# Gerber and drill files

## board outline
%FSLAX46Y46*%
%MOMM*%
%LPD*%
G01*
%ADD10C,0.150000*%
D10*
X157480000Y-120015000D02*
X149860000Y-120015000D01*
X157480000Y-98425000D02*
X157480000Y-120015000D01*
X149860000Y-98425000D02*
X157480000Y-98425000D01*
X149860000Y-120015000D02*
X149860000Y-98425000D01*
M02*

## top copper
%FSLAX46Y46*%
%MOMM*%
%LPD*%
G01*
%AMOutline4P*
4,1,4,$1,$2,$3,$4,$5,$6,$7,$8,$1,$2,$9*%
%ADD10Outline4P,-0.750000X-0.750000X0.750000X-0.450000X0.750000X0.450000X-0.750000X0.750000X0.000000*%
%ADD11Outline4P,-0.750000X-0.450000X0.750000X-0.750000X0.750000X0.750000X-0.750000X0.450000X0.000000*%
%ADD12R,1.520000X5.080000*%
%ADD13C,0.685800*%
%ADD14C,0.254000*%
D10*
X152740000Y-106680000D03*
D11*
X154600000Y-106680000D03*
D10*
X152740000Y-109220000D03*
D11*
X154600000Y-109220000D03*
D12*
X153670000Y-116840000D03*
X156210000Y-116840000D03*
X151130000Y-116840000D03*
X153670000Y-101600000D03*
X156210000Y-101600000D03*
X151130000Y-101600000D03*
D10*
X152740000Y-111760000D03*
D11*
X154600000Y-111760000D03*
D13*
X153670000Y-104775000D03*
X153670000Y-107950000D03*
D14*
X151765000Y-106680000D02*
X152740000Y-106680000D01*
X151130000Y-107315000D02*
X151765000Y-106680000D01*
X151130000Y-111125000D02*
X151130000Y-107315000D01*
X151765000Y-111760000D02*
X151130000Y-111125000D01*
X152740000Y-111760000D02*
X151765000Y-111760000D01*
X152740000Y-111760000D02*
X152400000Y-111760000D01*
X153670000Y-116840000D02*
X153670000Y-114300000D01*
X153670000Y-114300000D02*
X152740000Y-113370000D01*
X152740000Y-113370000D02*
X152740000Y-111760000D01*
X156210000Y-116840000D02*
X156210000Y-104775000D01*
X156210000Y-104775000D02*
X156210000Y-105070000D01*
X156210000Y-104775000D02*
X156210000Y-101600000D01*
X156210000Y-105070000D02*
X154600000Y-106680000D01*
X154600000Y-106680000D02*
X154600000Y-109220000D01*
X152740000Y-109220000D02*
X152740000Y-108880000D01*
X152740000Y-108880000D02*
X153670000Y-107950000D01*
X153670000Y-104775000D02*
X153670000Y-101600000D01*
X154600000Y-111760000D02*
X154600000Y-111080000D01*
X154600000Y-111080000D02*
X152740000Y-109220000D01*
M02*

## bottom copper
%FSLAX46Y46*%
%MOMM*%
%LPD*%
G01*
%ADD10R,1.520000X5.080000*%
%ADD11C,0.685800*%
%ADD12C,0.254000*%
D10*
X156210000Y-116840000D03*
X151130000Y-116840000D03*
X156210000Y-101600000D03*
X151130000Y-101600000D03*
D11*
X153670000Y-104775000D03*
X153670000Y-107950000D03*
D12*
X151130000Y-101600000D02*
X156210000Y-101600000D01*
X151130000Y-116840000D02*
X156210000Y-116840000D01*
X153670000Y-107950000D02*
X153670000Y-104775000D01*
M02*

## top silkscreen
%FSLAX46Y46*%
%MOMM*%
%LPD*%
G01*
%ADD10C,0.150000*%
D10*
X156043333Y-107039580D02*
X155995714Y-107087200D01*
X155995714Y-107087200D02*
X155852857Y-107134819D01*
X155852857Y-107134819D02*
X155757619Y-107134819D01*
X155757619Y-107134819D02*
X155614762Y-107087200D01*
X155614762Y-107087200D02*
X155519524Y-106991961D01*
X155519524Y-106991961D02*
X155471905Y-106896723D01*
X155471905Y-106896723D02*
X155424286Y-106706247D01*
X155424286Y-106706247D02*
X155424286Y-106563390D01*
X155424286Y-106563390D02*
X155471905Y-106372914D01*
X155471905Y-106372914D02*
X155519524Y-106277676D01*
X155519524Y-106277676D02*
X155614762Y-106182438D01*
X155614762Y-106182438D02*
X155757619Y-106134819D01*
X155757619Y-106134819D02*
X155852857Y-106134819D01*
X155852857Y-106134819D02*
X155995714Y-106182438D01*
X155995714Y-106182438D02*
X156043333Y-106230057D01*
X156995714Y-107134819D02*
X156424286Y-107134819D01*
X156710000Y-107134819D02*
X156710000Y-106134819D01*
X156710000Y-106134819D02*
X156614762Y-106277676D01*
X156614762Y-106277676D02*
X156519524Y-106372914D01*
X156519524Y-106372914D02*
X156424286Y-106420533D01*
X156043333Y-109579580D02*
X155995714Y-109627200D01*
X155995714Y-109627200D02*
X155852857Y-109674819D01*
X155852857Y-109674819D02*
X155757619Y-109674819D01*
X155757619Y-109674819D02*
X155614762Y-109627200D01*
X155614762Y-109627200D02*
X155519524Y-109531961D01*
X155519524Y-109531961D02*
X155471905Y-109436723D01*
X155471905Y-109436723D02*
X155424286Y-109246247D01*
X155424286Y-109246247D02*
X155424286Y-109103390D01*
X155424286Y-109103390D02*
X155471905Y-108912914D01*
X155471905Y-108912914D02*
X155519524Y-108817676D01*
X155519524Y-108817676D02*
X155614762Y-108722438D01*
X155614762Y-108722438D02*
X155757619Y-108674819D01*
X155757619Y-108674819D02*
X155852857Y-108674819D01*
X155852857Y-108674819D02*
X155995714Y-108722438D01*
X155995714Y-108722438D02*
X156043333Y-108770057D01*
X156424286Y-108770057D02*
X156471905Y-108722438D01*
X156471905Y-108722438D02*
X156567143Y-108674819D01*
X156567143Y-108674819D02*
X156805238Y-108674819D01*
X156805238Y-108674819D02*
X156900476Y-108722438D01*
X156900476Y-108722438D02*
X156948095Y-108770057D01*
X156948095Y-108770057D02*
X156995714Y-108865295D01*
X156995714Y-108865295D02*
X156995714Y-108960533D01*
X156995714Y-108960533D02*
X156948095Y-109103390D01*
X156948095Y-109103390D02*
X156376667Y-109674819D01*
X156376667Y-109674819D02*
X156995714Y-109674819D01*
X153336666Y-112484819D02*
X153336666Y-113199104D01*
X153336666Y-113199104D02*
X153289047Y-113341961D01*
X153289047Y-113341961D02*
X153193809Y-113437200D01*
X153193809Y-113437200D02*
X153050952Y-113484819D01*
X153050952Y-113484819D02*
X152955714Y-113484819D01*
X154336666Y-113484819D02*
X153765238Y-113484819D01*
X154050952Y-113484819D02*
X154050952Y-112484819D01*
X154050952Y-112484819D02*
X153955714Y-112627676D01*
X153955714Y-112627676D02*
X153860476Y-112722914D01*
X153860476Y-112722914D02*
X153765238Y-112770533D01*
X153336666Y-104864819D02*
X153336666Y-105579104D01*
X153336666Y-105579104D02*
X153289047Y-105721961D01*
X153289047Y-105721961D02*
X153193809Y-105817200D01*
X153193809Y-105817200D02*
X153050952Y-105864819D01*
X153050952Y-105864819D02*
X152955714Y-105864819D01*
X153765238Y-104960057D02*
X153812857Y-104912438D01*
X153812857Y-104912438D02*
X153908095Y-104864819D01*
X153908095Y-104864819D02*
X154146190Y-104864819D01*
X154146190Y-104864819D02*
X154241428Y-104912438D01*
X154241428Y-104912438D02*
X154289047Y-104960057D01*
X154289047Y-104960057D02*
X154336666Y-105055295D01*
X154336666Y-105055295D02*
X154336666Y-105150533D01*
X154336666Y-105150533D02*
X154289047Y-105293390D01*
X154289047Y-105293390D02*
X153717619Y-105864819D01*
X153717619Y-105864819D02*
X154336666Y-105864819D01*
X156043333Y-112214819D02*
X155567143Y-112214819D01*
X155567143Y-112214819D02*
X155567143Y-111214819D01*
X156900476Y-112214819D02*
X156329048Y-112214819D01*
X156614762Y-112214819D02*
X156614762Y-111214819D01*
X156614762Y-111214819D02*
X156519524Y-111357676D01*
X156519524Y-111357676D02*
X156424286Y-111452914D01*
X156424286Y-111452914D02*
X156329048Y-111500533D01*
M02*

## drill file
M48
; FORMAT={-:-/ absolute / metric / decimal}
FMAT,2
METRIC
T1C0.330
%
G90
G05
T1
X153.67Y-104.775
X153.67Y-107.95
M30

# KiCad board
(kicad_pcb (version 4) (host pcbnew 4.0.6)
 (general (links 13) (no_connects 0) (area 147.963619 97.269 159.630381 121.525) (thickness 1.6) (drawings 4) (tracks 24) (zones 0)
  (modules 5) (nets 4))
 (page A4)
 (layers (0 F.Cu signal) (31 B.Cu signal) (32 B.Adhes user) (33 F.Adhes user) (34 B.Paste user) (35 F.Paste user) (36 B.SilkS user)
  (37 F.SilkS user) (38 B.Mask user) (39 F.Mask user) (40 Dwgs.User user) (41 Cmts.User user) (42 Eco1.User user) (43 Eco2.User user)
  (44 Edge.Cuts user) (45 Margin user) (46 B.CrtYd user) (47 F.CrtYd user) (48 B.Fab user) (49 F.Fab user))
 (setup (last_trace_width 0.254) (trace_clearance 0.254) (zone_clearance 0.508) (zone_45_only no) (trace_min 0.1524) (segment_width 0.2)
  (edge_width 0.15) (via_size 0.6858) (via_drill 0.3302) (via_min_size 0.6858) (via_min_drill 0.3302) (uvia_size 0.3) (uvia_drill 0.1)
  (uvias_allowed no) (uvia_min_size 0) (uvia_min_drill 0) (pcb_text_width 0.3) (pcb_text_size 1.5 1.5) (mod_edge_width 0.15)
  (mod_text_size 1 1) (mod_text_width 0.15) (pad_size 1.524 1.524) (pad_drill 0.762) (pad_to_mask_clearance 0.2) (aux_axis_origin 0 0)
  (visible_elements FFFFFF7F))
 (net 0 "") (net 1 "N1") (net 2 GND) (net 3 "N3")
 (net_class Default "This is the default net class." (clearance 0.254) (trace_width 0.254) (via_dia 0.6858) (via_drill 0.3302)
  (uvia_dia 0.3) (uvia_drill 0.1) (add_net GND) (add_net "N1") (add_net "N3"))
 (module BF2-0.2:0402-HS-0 (layer F.Cu) (at 153.67 106.68)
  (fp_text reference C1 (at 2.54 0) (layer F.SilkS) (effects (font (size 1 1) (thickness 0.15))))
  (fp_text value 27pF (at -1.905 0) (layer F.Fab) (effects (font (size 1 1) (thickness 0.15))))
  (pad 1 smd trapezoid (at -0.93 0) (size 1.5 1.2) (rect_delta 0.3 0) (layers F.Cu F.Paste F.Mask) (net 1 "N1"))
  (pad 2 smd trapezoid (at 0.93 0) (size 1.5 1.2) (rect_delta -0.3 0) (layers F.Cu F.Paste F.Mask) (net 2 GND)))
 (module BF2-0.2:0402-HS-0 (layer F.Cu) (at 153.67 109.22)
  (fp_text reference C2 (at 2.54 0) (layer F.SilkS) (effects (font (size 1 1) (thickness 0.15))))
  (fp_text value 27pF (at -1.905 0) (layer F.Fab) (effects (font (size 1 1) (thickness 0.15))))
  (pad 1 smd trapezoid (at -0.93 0) (size 1.5 1.2) (rect_delta 0.3 0) (layers F.Cu F.Paste F.Mask) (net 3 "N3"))
  (pad 2 smd trapezoid (at 0.93 0) (size 1.5 1.2) (rect_delta -0.3 0) (layers F.Cu F.Paste F.Mask) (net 2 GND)))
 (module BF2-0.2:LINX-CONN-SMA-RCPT (layer F.Cu) (at 153.67 116.84)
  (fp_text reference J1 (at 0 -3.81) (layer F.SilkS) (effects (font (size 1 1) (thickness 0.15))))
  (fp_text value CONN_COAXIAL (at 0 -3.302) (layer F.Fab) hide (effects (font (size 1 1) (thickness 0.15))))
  (pad 1 smd rect (at 0 0) (size 1.52 5.08) (layers F.Cu F.Paste F.Mask) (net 1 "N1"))
  (pad 2 smd rect (at 2.54 0) (size 1.52 5.08) (layers F.Cu F.Paste F.Mask) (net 2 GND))
  (pad 2 smd rect (at -2.54 0) (size 1.52 5.08) (layers F.Cu F.Paste F.Mask) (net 2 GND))
  (pad 2 smd rect (at 2.54 0) (size 1.52 5.08) (layers B.Cu F.Paste F.Mask) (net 2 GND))
  (pad 2 smd rect (at -2.54 0) (size 1.52 5.08) (layers B.Cu F.Paste F.Mask) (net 2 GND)))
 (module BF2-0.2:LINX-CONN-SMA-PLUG (layer F.Cu) (at 153.67 101.6)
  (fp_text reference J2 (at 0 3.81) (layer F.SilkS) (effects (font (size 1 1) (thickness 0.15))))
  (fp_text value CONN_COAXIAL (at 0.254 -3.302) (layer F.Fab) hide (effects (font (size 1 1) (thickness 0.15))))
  (pad 1 smd rect (at 0 0) (size 1.52 5.08) (layers F.Cu F.Paste F.Mask) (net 3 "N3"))
  (pad 2 smd rect (at 2.54 0) (size 1.52 5.08) (layers F.Cu F.Paste F.Mask) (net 2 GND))
  (pad 2 smd rect (at -2.54 0) (size 1.52 5.08) (layers F.Cu F.Paste F.Mask) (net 2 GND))
  (pad 2 smd rect (at 2.54 0) (size 1.52 5.08) (layers B.Cu F.Paste F.Mask) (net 2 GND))
  (pad 2 smd rect (at -2.54 0) (size 1.52 5.08) (layers B.Cu F.Paste F.Mask) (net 2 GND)))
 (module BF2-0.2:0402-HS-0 (layer F.Cu) (at 153.67 111.76)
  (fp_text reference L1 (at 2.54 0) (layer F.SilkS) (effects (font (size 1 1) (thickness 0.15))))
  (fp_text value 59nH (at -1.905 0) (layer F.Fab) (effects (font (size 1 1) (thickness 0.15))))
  (pad 1 smd trapezoid (at -0.93 0) (size 1.5 1.2) (rect_delta 0.3 0) (layers F.Cu F.Paste F.Mask) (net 1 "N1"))
  (pad 2 smd trapezoid (at 0.93 0) (size 1.5 1.2) (rect_delta -0.3 0) (layers F.Cu F.Paste F.Mask) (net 3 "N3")))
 (gr_line (start 157.48 120.015) (end 149.86 120.015) (angle 90) (layer Edge.Cuts) (width 0.15))
 (gr_line (start 157.48 98.425) (end 157.48 120.015) (angle 90) (layer Edge.Cuts) (width 0.15))
 (gr_line (start 149.86 98.425) (end 157.48 98.425) (angle 90) (layer Edge.Cuts) (width 0.15))
 (gr_line (start 149.86 120.015) (end 149.86 98.425) (angle 90) (layer Edge.Cuts) (width 0.15))
 (segment (start 151.765 106.68) (end 152.74 106.68) (width 0.254) (layer F.Cu) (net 1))
 (segment (start 151.13 107.315) (end 151.765 106.68) (width 0.254) (layer F.Cu) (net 1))
 (segment (start 151.13 111.125) (end 151.13 107.315) (width 0.254) (layer F.Cu) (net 1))
 (segment (start 151.765 111.76) (end 151.13 111.125) (width 0.254) (layer F.Cu) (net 1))
 (segment (start 152.74 111.76) (end 151.765 111.76) (width 0.254) (layer F.Cu) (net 1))
 (segment (start 152.74 111.76) (end 152.4 111.76) (width 0.254) (layer F.Cu) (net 1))
 (segment (start 153.67 116.84) (end 153.67 114.3) (width 0.254) (layer F.Cu) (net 1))
 (segment (start 153.67 114.3) (end 152.74 113.37) (width 0.254) (layer F.Cu) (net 1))
 (segment (start 152.74 113.37) (end 152.74 111.76) (width 0.254) (layer F.Cu) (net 1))
 (segment (start 156.21 116.84) (end 156.21 104.775) (width 0.254) (layer F.Cu) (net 2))
 (segment (start 156.21 104.775) (end 156.21 105.07) (width 0.254) (layer F.Cu) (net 2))
 (segment (start 156.21 104.775) (end 156.21 101.6) (width 0.254) (layer F.Cu) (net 2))
 (segment (start 156.21 105.07) (end 154.6 106.68) (width 0.254) (layer F.Cu) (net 2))
 (segment (start 154.6 106.68) (end 154.6 109.22) (width 0.254) (layer F.Cu) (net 2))
 (segment (start 151.13 101.6) (end 156.21 101.6) (width 0.254) (layer B.Cu) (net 2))
 (segment (start 151.13 116.84) (end 156.21 116.84) (width 0.254) (layer B.Cu) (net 2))
 (segment (start 152.74 109.22) (end 152.74 108.88) (width 0.254) (layer F.Cu) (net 3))
 (segment (start 152.74 108.88) (end 153.67 107.95) (width 0.254) (layer F.Cu) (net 3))
 (segment (start 153.67 104.775) (end 153.67 101.6) (width 0.254) (layer F.Cu) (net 3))
 (via (at 153.67 104.775) (size 0.6858) (drill 0.3302) (layers F.Cu B.Cu) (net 3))
 (segment (start 153.67 107.95) (end 153.67 104.775) (width 0.254) (layer B.Cu) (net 3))
 (via (at 153.67 107.95) (size 0.6858) (drill 0.3302) (layers F.Cu B.Cu) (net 3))
 (segment (start 154.6 111.76) (end 154.6 111.08) (width 0.254) (layer F.Cu) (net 3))
 (segment (start 154.6 111.08) (end 152.74 109.22) (width 0.254) (layer F.Cu) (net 3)))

